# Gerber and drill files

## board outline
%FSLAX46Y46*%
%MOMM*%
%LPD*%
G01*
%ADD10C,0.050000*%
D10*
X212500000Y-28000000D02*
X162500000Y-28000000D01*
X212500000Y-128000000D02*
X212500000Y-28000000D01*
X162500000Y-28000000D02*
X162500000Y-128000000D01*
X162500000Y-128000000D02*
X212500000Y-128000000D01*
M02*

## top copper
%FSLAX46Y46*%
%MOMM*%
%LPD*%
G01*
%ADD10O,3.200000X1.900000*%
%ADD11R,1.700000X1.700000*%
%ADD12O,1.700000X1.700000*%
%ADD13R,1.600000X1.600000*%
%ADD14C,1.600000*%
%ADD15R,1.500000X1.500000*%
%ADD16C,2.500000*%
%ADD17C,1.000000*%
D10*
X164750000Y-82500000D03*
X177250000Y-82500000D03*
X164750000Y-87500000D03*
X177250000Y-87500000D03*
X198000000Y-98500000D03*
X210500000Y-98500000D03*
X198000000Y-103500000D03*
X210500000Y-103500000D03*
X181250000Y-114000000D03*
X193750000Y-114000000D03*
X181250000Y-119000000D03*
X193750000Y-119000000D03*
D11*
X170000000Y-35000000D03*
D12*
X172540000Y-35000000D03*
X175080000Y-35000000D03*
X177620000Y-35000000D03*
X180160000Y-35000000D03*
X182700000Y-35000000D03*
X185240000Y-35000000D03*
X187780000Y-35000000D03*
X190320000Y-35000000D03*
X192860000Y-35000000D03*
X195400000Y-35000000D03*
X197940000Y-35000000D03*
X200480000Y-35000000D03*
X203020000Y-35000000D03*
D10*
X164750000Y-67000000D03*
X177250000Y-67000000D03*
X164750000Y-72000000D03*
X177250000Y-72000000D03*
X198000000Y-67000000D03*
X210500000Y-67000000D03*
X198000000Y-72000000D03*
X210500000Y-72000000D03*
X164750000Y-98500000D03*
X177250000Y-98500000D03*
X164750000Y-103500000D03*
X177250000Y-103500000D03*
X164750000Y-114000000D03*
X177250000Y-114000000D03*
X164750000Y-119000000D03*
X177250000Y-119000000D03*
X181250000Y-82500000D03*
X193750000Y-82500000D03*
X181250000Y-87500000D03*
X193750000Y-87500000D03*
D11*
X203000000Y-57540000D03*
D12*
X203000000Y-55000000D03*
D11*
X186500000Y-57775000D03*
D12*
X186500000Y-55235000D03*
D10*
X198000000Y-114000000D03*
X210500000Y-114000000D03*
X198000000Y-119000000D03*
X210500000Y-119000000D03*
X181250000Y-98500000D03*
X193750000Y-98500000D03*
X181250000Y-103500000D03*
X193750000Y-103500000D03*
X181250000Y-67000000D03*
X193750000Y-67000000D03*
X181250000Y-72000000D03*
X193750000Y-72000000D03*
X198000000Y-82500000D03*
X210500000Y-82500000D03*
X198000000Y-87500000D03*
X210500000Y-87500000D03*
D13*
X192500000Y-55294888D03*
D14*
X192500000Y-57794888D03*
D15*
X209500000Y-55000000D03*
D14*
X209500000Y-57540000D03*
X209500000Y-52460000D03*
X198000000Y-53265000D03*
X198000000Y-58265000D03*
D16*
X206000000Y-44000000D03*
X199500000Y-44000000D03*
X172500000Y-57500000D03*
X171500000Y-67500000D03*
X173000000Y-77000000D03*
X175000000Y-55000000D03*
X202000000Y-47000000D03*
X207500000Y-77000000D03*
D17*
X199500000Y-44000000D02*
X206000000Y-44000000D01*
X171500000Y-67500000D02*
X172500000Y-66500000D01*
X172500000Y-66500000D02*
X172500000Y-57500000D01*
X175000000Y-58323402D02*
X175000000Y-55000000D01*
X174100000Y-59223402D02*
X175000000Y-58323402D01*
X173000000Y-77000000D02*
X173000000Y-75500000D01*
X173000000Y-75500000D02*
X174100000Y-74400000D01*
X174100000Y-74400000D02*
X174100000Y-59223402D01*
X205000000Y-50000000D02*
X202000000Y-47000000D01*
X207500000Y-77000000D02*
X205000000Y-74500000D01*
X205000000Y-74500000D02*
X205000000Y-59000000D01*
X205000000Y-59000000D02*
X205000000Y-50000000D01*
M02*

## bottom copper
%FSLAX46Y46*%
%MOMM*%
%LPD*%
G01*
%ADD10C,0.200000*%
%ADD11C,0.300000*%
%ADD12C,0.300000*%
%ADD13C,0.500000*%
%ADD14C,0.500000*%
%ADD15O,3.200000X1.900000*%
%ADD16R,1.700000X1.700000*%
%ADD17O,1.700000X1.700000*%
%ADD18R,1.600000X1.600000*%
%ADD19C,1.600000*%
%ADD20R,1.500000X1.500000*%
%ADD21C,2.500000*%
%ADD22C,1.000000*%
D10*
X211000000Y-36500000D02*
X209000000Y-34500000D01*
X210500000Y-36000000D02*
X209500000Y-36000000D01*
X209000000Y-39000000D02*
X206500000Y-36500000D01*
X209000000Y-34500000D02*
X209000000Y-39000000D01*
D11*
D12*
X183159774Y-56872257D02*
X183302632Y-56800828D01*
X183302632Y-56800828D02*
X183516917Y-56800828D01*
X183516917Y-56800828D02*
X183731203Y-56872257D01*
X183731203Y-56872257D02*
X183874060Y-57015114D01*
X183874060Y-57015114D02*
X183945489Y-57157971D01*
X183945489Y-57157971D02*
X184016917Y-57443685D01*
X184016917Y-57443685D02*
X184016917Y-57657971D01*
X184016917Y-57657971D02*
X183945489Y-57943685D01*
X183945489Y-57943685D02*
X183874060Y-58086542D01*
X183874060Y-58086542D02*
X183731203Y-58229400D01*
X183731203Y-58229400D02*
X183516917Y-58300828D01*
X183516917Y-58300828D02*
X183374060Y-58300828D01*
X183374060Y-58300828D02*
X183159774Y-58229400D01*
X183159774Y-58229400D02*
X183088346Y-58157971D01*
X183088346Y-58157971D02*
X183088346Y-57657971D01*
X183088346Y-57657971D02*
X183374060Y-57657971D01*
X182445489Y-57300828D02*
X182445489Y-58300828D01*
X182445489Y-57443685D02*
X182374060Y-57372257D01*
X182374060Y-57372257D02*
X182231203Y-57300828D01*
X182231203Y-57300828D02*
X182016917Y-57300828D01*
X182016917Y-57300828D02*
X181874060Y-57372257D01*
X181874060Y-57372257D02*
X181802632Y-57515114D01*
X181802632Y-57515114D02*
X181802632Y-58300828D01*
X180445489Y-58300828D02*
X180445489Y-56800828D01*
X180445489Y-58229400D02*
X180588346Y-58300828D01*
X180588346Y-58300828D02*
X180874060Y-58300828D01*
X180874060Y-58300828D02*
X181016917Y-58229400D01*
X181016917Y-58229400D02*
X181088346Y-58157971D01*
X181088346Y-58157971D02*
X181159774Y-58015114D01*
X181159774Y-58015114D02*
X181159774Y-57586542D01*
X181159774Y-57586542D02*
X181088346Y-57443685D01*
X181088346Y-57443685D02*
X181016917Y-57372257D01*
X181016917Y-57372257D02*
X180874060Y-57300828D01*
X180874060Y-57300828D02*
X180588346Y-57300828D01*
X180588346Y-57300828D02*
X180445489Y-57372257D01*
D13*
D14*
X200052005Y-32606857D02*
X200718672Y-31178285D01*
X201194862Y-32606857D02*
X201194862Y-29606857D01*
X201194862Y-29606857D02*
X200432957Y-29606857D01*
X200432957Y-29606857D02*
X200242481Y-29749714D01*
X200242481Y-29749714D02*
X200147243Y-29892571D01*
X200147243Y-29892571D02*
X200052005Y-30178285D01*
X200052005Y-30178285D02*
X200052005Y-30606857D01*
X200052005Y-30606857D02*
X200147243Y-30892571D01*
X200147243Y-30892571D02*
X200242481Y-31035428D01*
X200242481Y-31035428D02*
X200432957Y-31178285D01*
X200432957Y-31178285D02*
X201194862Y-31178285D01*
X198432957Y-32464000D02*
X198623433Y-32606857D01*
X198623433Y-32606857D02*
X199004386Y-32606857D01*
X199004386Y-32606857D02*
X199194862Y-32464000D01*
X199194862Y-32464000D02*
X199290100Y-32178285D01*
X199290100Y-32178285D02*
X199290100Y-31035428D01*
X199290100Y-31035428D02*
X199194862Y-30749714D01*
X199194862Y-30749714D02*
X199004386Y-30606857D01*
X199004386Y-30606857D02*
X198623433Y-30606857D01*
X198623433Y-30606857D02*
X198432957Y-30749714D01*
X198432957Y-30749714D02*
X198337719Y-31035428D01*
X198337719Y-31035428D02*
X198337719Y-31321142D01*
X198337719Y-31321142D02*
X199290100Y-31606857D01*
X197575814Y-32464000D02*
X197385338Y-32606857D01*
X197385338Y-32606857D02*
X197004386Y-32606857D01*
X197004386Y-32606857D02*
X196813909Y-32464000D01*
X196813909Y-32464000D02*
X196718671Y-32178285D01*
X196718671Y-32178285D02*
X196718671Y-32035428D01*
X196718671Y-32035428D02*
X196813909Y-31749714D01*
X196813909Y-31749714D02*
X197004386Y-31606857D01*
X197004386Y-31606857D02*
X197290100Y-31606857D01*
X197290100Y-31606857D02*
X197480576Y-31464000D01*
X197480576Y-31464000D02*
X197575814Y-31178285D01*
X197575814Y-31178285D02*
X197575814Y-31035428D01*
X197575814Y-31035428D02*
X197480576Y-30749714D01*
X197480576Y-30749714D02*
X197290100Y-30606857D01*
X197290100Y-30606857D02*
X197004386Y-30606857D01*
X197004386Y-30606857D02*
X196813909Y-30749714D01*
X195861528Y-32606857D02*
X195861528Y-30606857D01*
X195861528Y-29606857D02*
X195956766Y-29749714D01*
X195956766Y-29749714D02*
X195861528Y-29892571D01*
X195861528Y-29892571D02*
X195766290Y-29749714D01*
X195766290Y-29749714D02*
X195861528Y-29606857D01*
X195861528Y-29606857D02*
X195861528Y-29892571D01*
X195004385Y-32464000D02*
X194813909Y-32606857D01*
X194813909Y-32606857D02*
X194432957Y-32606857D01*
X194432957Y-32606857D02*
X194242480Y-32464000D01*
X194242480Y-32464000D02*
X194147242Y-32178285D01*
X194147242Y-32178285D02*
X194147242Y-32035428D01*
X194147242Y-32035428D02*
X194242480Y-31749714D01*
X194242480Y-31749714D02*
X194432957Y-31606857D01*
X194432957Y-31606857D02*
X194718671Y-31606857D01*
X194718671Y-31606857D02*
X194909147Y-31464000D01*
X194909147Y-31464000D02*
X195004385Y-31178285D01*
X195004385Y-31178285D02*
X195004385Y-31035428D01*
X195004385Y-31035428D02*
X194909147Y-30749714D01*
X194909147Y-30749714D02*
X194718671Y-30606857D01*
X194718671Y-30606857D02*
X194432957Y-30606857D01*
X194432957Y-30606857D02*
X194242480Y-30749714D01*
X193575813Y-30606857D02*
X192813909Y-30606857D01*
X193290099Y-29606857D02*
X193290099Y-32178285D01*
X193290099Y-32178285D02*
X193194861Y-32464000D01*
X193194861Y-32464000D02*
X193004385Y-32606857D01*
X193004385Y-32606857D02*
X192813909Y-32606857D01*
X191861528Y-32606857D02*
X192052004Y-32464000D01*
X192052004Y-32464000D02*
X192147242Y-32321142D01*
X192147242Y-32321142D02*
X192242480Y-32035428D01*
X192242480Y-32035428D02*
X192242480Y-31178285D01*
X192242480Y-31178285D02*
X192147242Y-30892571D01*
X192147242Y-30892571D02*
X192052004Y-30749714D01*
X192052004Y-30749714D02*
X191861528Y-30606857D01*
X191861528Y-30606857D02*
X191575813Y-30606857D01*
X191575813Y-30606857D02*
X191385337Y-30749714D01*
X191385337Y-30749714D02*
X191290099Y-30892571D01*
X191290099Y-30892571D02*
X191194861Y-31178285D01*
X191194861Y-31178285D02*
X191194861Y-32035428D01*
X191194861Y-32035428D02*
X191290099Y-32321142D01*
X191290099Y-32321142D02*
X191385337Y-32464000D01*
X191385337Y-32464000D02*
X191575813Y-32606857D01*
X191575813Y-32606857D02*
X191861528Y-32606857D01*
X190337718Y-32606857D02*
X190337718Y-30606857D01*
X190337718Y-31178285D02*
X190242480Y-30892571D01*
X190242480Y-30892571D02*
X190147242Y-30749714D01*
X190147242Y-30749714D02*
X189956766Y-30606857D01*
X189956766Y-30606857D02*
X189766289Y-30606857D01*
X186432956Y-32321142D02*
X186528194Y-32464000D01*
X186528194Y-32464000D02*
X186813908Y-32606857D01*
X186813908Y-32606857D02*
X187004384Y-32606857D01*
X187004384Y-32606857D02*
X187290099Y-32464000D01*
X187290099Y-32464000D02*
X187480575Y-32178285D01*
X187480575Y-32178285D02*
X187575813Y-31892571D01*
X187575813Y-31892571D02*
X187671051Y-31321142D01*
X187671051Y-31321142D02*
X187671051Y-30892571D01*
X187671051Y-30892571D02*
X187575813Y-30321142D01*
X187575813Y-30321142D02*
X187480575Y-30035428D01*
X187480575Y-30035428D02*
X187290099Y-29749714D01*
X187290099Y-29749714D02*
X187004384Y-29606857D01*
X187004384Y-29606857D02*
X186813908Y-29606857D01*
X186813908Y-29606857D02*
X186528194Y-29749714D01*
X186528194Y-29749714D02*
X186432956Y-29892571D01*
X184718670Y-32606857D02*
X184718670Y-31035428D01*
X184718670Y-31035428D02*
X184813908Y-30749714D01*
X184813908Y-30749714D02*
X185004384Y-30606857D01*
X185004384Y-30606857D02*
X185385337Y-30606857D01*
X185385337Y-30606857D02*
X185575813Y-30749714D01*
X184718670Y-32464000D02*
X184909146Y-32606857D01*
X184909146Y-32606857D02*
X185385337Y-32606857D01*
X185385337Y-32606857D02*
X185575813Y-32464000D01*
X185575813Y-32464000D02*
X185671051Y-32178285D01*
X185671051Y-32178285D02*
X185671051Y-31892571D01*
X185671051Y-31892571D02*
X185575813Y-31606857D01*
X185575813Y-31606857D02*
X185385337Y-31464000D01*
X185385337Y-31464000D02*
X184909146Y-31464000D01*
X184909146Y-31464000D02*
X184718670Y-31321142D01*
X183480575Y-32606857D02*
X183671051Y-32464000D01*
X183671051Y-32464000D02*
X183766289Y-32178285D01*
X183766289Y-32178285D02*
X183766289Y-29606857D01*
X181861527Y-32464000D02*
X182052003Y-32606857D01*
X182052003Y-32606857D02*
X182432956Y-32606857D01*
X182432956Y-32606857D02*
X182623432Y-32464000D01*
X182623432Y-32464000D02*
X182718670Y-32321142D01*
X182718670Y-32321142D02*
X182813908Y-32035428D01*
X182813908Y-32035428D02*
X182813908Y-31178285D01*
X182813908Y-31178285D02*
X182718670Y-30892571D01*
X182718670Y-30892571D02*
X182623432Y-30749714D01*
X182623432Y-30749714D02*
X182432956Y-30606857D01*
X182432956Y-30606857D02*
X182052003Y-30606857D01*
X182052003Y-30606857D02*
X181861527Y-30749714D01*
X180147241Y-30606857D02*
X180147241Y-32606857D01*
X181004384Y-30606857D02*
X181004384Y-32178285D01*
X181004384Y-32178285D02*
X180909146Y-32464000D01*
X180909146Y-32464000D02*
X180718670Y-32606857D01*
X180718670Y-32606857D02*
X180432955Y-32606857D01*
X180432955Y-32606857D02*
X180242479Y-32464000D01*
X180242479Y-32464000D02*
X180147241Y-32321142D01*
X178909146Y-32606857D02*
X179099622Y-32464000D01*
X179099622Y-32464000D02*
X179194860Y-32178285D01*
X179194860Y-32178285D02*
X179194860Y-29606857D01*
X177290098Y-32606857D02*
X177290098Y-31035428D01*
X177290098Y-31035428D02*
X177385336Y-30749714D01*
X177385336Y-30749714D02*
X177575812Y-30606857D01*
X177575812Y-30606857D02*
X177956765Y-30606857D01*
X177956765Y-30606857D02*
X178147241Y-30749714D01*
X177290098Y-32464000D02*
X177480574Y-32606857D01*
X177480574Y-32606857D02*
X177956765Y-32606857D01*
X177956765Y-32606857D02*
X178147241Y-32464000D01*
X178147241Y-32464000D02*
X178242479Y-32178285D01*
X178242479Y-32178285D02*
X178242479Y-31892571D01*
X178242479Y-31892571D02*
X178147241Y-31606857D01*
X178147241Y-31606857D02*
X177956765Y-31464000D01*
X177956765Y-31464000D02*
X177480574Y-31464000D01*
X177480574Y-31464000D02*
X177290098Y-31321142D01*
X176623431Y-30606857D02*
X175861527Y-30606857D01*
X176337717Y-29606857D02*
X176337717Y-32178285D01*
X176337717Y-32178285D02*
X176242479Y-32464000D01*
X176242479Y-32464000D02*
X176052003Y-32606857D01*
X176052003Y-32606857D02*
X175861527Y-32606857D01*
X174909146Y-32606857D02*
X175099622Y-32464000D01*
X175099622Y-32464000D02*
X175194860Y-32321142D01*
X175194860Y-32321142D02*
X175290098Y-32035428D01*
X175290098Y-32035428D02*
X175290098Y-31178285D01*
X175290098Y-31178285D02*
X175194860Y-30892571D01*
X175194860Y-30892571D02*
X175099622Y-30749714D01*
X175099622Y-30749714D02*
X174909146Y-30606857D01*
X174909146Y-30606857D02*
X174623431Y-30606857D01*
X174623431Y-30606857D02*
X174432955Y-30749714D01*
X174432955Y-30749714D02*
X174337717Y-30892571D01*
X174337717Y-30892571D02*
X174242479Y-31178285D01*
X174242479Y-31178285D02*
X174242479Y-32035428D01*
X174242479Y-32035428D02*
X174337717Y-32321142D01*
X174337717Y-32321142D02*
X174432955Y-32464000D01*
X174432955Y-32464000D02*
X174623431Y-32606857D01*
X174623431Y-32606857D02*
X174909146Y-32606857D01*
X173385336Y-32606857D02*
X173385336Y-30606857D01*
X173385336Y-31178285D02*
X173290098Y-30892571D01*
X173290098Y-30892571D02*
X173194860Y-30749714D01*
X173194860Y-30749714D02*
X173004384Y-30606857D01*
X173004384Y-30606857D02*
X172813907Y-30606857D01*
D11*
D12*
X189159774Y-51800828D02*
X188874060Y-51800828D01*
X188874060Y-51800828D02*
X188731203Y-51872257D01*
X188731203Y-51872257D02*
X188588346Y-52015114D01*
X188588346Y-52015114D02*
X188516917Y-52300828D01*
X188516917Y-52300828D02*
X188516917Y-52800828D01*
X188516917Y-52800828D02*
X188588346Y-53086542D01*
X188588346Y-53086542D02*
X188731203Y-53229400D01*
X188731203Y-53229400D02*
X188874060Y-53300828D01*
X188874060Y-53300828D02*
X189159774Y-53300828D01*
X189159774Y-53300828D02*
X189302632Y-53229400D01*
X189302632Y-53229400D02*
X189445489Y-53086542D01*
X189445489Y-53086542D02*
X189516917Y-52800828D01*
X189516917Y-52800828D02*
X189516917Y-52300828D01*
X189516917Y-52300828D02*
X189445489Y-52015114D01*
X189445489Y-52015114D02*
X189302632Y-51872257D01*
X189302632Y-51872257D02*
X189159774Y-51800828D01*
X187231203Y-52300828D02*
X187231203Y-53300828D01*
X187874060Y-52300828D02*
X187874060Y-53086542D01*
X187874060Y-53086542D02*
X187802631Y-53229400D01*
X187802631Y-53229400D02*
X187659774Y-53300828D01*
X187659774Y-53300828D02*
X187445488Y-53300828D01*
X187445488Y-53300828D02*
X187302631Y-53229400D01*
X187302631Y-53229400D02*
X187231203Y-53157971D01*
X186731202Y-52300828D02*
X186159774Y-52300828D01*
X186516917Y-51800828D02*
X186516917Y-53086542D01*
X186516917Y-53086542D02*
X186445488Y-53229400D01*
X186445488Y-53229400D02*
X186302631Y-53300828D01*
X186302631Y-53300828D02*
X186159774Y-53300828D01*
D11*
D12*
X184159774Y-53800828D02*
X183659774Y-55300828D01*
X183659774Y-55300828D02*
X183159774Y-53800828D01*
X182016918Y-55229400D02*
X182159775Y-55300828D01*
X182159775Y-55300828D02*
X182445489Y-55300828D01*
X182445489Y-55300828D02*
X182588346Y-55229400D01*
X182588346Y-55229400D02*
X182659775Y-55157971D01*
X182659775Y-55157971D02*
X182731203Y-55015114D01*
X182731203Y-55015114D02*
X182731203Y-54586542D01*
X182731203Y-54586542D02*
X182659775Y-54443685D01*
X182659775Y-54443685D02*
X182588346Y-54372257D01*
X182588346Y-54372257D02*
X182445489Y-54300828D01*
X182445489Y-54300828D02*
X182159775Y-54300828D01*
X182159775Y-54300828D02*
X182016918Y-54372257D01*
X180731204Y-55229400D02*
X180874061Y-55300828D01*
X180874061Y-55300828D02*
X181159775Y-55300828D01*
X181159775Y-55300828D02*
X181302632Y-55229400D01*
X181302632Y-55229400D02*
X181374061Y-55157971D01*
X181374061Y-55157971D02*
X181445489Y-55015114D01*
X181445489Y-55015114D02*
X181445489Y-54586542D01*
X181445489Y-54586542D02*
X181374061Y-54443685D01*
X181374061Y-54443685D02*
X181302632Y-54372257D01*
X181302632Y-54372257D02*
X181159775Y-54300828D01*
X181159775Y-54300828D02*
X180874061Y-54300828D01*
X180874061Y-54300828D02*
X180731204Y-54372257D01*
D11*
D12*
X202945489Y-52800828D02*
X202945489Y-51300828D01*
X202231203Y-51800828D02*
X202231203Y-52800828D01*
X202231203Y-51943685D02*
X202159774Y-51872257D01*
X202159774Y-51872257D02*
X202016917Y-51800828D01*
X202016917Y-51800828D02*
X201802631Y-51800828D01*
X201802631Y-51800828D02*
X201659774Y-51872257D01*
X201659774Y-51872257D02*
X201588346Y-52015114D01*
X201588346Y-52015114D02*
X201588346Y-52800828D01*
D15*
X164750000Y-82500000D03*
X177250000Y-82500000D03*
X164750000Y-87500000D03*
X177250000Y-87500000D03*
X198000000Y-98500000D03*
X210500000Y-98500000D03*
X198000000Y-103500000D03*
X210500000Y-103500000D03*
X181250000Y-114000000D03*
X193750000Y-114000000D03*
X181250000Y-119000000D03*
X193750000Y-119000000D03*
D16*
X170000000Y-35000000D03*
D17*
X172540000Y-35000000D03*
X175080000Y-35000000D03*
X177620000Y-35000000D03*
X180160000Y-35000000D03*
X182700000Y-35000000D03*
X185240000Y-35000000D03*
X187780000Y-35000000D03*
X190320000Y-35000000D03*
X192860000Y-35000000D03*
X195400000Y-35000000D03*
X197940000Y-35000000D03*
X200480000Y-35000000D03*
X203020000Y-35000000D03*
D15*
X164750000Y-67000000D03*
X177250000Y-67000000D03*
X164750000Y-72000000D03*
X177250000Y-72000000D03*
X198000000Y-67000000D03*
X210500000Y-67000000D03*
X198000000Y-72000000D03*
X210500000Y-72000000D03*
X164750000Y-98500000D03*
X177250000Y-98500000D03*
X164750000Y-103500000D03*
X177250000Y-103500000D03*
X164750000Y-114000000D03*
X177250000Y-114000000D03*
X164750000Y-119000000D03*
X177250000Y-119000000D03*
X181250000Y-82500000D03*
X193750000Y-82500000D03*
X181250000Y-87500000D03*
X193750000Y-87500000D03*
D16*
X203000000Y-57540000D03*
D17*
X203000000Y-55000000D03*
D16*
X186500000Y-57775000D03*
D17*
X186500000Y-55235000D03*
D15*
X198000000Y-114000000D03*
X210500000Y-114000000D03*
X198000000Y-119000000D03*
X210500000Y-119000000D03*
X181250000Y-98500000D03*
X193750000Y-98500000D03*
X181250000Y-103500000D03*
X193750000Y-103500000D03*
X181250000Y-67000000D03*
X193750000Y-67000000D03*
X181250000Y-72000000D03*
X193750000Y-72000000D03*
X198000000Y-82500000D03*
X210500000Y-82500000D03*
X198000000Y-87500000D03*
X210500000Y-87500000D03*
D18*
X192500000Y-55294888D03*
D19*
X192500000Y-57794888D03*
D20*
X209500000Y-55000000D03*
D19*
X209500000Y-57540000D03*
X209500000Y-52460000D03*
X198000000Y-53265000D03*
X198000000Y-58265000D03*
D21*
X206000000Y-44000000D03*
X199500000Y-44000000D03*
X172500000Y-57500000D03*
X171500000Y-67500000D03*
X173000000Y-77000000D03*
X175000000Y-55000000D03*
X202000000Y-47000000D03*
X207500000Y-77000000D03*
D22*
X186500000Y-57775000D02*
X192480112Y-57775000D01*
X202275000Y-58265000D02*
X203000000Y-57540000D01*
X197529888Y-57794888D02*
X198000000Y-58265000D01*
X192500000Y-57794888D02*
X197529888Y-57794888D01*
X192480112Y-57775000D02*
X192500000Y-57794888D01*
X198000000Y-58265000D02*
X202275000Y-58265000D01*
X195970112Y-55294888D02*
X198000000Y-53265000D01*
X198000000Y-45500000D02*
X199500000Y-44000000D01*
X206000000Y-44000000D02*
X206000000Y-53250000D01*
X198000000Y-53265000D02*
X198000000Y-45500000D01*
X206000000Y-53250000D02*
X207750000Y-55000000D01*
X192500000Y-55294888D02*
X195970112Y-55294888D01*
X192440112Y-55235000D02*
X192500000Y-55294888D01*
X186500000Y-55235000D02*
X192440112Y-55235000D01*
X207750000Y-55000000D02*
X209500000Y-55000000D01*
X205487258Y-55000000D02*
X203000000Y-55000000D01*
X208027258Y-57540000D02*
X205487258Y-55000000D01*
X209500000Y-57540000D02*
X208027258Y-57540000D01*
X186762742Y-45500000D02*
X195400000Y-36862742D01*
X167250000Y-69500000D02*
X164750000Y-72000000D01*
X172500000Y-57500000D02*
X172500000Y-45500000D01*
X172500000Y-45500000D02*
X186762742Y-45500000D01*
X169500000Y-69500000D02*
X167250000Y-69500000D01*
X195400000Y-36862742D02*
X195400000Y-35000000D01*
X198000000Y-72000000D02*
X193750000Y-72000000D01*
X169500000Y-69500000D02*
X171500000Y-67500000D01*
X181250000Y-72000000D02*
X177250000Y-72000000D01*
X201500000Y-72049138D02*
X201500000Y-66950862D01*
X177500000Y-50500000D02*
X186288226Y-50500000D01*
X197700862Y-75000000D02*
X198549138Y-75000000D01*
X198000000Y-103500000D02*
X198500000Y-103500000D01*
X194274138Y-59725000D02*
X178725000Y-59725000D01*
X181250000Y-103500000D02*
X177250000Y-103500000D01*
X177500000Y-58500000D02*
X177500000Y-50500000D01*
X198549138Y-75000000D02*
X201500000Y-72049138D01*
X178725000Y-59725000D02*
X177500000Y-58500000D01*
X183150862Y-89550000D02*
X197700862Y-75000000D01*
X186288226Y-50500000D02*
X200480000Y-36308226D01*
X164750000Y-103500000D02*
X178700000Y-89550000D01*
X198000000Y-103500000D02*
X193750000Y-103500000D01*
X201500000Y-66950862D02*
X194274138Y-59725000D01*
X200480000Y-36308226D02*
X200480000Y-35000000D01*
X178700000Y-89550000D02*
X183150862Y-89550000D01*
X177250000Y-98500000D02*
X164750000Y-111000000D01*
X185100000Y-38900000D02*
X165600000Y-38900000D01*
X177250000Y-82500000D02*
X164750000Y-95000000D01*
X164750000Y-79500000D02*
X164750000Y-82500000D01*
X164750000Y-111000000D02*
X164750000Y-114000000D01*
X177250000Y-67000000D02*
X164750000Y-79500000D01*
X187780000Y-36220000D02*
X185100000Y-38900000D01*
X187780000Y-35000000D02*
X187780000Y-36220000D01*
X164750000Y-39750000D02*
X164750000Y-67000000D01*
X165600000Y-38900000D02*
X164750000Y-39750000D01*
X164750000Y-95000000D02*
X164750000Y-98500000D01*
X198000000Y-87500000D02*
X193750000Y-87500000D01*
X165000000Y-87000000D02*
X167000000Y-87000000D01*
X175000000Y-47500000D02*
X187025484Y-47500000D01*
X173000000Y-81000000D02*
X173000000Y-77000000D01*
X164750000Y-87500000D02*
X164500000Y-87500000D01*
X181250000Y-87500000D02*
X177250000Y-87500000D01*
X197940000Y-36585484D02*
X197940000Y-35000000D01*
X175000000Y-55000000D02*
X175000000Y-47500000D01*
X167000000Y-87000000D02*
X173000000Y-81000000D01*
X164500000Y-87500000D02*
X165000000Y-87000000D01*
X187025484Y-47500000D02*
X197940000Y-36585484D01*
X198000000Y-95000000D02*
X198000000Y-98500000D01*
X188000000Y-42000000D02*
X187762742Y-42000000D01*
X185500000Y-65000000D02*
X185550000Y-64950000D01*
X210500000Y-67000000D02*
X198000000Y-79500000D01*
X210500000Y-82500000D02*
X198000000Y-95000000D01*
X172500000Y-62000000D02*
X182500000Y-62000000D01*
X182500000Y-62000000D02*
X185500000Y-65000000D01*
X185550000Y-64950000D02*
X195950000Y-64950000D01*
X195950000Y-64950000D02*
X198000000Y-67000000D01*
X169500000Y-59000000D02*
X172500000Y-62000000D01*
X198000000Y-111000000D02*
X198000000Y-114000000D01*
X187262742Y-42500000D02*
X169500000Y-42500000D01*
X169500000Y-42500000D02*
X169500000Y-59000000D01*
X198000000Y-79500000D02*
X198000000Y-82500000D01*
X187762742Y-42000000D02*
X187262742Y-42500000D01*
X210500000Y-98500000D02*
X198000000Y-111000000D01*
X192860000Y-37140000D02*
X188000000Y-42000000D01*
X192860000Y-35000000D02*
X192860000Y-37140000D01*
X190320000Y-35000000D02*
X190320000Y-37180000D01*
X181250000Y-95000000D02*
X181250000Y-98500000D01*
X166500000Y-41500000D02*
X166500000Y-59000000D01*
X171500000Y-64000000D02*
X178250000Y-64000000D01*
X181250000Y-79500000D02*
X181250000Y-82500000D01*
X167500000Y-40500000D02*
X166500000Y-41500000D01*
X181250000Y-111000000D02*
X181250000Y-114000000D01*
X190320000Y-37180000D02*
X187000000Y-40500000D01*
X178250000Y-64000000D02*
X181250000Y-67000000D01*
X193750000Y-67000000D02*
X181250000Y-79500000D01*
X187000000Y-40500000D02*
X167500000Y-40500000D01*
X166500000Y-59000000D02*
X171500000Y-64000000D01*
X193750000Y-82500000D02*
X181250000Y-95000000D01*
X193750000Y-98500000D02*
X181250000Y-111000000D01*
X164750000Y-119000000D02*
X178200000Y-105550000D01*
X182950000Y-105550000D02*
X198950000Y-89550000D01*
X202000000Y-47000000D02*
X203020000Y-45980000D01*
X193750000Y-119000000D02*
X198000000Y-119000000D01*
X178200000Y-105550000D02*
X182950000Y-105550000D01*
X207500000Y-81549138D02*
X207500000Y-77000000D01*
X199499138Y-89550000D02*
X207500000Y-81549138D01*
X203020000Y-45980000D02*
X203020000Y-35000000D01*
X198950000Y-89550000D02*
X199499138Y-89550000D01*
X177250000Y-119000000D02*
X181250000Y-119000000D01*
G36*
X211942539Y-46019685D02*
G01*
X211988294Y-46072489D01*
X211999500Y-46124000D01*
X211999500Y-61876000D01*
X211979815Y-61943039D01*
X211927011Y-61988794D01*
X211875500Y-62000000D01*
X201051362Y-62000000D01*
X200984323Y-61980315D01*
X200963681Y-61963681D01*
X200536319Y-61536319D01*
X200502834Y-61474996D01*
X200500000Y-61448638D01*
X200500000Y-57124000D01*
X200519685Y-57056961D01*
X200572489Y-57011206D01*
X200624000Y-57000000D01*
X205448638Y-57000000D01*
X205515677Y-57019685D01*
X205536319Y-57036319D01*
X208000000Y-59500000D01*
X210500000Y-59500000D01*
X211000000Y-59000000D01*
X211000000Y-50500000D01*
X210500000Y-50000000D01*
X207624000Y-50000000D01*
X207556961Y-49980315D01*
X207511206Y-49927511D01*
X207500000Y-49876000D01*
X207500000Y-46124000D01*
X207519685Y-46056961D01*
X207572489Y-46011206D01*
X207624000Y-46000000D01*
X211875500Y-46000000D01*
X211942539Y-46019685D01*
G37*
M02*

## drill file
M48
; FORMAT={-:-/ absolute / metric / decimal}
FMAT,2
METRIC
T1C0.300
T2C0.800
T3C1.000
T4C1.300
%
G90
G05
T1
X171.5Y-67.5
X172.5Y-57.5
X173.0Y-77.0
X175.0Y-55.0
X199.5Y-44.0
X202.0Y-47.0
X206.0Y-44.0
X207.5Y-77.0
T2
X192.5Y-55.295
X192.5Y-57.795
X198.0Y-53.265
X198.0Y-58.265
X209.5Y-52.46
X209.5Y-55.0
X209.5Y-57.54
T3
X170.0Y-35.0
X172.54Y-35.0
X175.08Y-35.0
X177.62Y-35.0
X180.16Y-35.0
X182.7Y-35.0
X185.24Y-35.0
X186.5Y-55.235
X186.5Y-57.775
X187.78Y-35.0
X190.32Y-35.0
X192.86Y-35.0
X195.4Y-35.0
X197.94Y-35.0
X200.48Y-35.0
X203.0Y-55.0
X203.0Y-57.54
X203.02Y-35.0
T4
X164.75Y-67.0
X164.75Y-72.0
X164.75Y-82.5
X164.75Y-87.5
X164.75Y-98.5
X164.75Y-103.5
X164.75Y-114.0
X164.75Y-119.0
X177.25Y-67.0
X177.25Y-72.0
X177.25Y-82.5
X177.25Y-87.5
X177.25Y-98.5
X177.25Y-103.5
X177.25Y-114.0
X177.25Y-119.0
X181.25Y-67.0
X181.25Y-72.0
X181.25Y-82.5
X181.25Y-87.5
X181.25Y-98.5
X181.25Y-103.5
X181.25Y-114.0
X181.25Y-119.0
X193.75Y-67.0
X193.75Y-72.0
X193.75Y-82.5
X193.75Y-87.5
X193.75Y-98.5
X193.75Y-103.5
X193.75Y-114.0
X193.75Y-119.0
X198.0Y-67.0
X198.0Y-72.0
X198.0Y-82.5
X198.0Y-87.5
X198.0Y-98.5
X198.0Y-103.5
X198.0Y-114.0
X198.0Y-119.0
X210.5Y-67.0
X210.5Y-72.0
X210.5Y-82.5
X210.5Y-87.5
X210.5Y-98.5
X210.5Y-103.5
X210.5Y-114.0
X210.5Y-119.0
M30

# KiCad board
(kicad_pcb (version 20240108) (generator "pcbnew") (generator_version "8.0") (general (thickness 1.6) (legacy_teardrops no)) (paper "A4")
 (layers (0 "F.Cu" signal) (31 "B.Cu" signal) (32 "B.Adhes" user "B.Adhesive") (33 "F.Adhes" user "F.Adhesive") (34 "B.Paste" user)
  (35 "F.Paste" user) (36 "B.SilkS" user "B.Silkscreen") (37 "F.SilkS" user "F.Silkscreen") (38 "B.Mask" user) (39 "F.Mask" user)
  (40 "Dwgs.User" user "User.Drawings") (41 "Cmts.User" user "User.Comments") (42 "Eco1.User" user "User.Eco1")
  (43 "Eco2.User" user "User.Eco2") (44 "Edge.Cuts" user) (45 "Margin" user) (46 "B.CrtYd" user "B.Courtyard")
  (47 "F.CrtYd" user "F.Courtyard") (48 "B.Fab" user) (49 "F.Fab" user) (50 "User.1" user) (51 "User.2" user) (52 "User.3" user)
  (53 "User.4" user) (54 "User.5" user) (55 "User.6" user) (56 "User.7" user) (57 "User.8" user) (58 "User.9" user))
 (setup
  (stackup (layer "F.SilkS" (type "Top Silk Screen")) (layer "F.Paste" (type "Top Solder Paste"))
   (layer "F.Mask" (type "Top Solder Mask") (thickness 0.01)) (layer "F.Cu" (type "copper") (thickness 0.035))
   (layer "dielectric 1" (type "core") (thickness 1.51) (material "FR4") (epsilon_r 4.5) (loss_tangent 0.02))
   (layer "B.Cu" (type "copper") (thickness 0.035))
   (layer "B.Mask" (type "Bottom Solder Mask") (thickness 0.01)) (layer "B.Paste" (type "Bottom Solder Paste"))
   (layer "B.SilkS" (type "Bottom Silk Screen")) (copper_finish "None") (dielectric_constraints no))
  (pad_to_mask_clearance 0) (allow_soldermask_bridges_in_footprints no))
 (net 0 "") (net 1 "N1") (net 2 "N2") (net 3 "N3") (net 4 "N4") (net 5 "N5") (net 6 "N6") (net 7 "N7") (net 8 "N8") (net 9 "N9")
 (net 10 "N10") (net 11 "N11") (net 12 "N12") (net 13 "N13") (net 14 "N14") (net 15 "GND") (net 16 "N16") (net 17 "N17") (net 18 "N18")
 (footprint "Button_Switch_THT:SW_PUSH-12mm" (layer "F.Cu") (at 164.75 82.5)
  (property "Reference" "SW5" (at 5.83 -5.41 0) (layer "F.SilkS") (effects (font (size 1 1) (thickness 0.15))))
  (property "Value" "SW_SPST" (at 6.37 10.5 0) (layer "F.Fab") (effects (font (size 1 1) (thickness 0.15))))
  (pad "1" thru_hole oval (at 0 0) (size 3.2 1.9) (drill 1.3) (layers "*.Cu" "*.Mask") (remove_unused_layers no) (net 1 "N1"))
  (pad "1" thru_hole oval (at 12.5 0) (size 3.2 1.9) (drill 1.3) (layers "*.Cu" "*.Mask") (remove_unused_layers no) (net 1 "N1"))
  (pad "2" thru_hole oval (at 0 5) (size 3.2 1.9) (drill 1.3) (layers "*.Cu" "*.Mask") (remove_unused_layers no) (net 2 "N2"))
  (pad "2" thru_hole oval (at 12.5 5) (size 3.2 1.9) (drill 1.3) (layers "*.Cu" "*.Mask") (remove_unused_layers no) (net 2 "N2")))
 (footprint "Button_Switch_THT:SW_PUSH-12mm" (layer "F.Cu") (at 198 98.5)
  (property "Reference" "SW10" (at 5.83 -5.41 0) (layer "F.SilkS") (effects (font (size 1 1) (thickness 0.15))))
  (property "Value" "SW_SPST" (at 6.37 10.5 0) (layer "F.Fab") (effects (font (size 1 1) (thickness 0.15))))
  (pad "1" thru_hole oval (at 0 0) (size 3.2 1.9) (drill 1.3) (layers "*.Cu" "*.Mask") (remove_unused_layers no) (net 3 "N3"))
  (pad "1" thru_hole oval (at 12.5 0) (size 3.2 1.9) (drill 1.3) (layers "*.Cu" "*.Mask") (remove_unused_layers no) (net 3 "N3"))
  (pad "2" thru_hole oval (at 0 5) (size 3.2 1.9) (drill 1.3) (layers "*.Cu" "*.Mask") (remove_unused_layers no) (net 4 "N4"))
  (pad "2" thru_hole oval (at 12.5 5) (size 3.2 1.9) (drill 1.3) (layers "*.Cu" "*.Mask") (remove_unused_layers no) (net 4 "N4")))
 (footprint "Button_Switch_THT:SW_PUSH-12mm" (layer "F.Cu") (at 181.25 114)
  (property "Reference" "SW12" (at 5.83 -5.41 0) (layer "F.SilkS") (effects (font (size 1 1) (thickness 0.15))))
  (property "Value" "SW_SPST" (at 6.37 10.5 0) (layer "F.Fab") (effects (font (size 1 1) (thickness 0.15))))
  (pad "1" thru_hole oval (at 0 0) (size 3.2 1.9) (drill 1.3) (layers "*.Cu" "*.Mask") (remove_unused_layers no) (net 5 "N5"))
  (pad "1" thru_hole oval (at 12.5 0) (size 3.2 1.9) (drill 1.3) (layers "*.Cu" "*.Mask") (remove_unused_layers no) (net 5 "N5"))
  (pad "2" thru_hole oval (at 0 5) (size 3.2 1.9) (drill 1.3) (layers "*.Cu" "*.Mask") (remove_unused_layers no) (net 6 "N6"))
  (pad "2" thru_hole oval (at 12.5 5) (size 3.2 1.9) (drill 1.3) (layers "*.Cu" "*.Mask") (remove_unused_layers no) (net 6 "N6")))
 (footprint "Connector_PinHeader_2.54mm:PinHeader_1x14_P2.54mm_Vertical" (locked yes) (layer "F.Cu") (at 170 35 90)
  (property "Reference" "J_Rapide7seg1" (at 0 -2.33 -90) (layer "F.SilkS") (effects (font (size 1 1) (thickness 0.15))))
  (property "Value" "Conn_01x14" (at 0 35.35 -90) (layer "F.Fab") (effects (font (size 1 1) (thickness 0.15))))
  (pad "1" thru_hole rect (at 0 0 90) (size 1.7 1.7) (drill 1) (layers "*.Cu" "*.Mask") (remove_unused_layers no) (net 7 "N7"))
  (pad "2" thru_hole oval (at 0 2.54 90) (size 1.7 1.7) (drill 1) (layers "*.Cu" "*.Mask") (remove_unused_layers no) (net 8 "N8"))
  (pad "3" thru_hole oval (at 0 5.08 90) (size 1.7 1.7) (drill 1) (layers "*.Cu" "*.Mask") (remove_unused_layers no) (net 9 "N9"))
  (pad "4" thru_hole oval (at 0 7.62 90) (size 1.7 1.7) (drill 1) (layers "*.Cu" "*.Mask") (remove_unused_layers no) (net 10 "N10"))
  (pad "5" thru_hole oval (at 0 10.16 90) (size 1.7 1.7) (drill 1) (layers "*.Cu" "*.Mask") (remove_unused_layers no) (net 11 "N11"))
  (pad "6" thru_hole oval (at 0 12.7 90) (size 1.7 1.7) (drill 1) (layers "*.Cu" "*.Mask") (remove_unused_layers no) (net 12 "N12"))
  (pad "7" thru_hole oval (at 0 15.24 90) (size 1.7 1.7) (drill 1) (layers "*.Cu" "*.Mask") (remove_unused_layers no) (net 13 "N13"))
  (pad "8" thru_hole oval (at 0 17.78 90) (size 1.7 1.7) (drill 1) (layers "*.Cu" "*.Mask") (remove_unused_layers no) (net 1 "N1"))
  (pad "9" thru_hole oval (at 0 20.32 90) (size 1.7 1.7) (drill 1) (layers "*.Cu" "*.Mask") (remove_unused_layers no) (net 5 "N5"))
  (pad "10" thru_hole oval (at 0 22.86 90) (size 1.7 1.7) (drill 1) (layers "*.Cu" "*.Mask") (remove_unused_layers no) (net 3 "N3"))
  (pad "11" thru_hole oval (at 0 25.4 90) (size 1.7 1.7) (drill 1) (layers "*.Cu" "*.Mask") (remove_unused_layers no) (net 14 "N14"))
  (pad "12" thru_hole oval (at 0 27.94 90) (size 1.7 1.7) (drill 1) (layers "*.Cu" "*.Mask") (remove_unused_layers no) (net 2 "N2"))
  (pad "13" thru_hole oval (at 0 30.48 90) (size 1.7 1.7) (drill 1) (layers "*.Cu" "*.Mask") (remove_unused_layers no) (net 4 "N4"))
  (pad "14" thru_hole oval (at 0 33.02 90) (size 1.7 1.7) (drill 1) (layers "*.Cu" "*.Mask") (remove_unused_layers no) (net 6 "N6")))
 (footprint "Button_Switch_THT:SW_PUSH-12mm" (layer "F.Cu") (at 164.75 67)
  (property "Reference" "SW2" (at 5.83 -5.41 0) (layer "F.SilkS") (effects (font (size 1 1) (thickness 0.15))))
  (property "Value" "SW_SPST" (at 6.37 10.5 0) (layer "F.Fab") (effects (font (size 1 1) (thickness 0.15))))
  (pad "1" thru_hole oval (at 0 0) (size 3.2 1.9) (drill 1.3) (layers "*.Cu" "*.Mask") (remove_unused_layers no) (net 1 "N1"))
  (pad "1" thru_hole oval (at 12.5 0) (size 3.2 1.9) (drill 1.3) (layers "*.Cu" "*.Mask") (remove_unused_layers no) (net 1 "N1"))
  (pad "2" thru_hole oval (at 0 5) (size 3.2 1.9) (drill 1.3) (layers "*.Cu" "*.Mask") (remove_unused_layers no) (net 14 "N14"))
  (pad "2" thru_hole oval (at 12.5 5) (size 3.2 1.9) (drill 1.3) (layers "*.Cu" "*.Mask") (remove_unused_layers no) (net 14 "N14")))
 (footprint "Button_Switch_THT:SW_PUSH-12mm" (layer "F.Cu") (at 198 67)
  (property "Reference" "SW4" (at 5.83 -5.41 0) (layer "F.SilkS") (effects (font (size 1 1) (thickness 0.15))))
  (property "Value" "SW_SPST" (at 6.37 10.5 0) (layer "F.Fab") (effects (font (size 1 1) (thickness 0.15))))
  (pad "1" thru_hole oval (at 0 0) (size 3.2 1.9) (drill 1.3) (layers "*.Cu" "*.Mask") (remove_unused_layers no) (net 3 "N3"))
  (pad "1" thru_hole oval (at 12.5 0) (size 3.2 1.9) (drill 1.3) (layers "*.Cu" "*.Mask") (remove_unused_layers no) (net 3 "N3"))
  (pad "2" thru_hole oval (at 0 5) (size 3.2 1.9) (drill 1.3) (layers "*.Cu" "*.Mask") (remove_unused_layers no) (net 14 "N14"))
  (pad "2" thru_hole oval (at 12.5 5) (size 3.2 1.9) (drill 1.3) (layers "*.Cu" "*.Mask") (remove_unused_layers no) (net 14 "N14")))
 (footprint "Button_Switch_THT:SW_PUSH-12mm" (layer "F.Cu") (at 164.75 98.5)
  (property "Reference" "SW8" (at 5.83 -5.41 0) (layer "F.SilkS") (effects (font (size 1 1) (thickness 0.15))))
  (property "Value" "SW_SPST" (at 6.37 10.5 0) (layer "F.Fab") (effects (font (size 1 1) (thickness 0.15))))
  (pad "1" thru_hole oval (at 0 0) (size 3.2 1.9) (drill 1.3) (layers "*.Cu" "*.Mask") (remove_unused_layers no) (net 1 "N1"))
  (pad "1" thru_hole oval (at 12.5 0) (size 3.2 1.9) (drill 1.3) (layers "*.Cu" "*.Mask") (remove_unused_layers no) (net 1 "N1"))
  (pad "2" thru_hole oval (at 0 5) (size 3.2 1.9) (drill 1.3) (layers "*.Cu" "*.Mask") (remove_unused_layers no) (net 4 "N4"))
  (pad "2" thru_hole oval (at 12.5 5) (size 3.2 1.9) (drill 1.3) (layers "*.Cu" "*.Mask") (remove_unused_layers no) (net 4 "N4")))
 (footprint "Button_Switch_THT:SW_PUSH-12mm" (layer "F.Cu") (at 164.75 114)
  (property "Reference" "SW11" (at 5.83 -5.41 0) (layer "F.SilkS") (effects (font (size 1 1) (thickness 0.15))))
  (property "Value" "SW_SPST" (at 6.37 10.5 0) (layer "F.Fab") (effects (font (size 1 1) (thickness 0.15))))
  (pad "1" thru_hole oval (at 0 0) (size 3.2 1.9) (drill 1.3) (layers "*.Cu" "*.Mask") (remove_unused_layers no) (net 1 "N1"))
  (pad "1" thru_hole oval (at 12.5 0) (size 3.2 1.9) (drill 1.3) (layers "*.Cu" "*.Mask") (remove_unused_layers no) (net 1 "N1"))
  (pad "2" thru_hole oval (at 0 5) (size 3.2 1.9) (drill 1.3) (layers "*.Cu" "*.Mask") (remove_unused_layers no) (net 6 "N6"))
  (pad "2" thru_hole oval (at 12.5 5) (size 3.2 1.9) (drill 1.3) (layers "*.Cu" "*.Mask") (remove_unused_layers no) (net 6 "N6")))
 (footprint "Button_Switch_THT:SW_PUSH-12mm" (layer "F.Cu") (at 181.25 82.5)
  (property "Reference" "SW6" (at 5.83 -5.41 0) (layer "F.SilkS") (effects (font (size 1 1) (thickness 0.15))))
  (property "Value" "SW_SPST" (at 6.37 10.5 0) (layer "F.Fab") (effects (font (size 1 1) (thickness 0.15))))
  (pad "1" thru_hole oval (at 0 0) (size 3.2 1.9) (drill 1.3) (layers "*.Cu" "*.Mask") (remove_unused_layers no) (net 5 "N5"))
  (pad "1" thru_hole oval (at 12.5 0) (size 3.2 1.9) (drill 1.3) (layers "*.Cu" "*.Mask") (remove_unused_layers no) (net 5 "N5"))
  (pad "2" thru_hole oval (at 0 5) (size 3.2 1.9) (drill 1.3) (layers "*.Cu" "*.Mask") (remove_unused_layers no) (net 2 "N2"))
  (pad "2" thru_hole oval (at 12.5 5) (size 3.2 1.9) (drill 1.3) (layers "*.Cu" "*.Mask") (remove_unused_layers no) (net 2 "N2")))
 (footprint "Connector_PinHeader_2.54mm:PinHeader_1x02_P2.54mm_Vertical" (layer "F.Cu") (at 203 57.54 180)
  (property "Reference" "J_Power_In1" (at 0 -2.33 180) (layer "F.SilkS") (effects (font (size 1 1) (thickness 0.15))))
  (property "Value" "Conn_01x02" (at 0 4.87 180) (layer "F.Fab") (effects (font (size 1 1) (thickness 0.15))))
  (pad "1" thru_hole rect (at 0 0 180) (size 1.7 1.7) (drill 1) (layers "*.Cu" "*.Mask") (remove_unused_layers no) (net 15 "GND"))
  (pad "2" thru_hole oval (at 0 2.54 180) (size 1.7 1.7) (drill 1) (layers "*.Cu" "*.Mask") (remove_unused_layers no) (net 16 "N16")))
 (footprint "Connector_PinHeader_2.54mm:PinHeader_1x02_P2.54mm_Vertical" (layer "F.Cu") (at 186.5 57.775 180)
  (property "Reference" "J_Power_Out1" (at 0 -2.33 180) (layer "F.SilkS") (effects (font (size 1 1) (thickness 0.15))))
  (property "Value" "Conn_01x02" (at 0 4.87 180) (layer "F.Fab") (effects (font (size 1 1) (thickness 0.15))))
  (pad "1" thru_hole rect (at 0 0 180) (size 1.7 1.7) (drill 1) (layers "*.Cu" "*.Mask") (remove_unused_layers no) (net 15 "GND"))
  (pad "2" thru_hole oval (at 0 2.54 180) (size 1.7 1.7) (drill 1) (layers "*.Cu" "*.Mask") (remove_unused_layers no) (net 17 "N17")))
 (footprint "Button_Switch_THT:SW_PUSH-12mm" (layer "F.Cu") (at 198 114)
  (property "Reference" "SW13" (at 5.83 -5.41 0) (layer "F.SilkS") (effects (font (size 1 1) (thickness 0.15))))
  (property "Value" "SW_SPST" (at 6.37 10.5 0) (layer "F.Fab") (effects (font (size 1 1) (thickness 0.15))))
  (pad "1" thru_hole oval (at 0 0) (size 3.2 1.9) (drill 1.3) (layers "*.Cu" "*.Mask") (remove_unused_layers no) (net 3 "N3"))
  (pad "1" thru_hole oval (at 12.5 0) (size 3.2 1.9) (drill 1.3) (layers "*.Cu" "*.Mask") (remove_unused_layers no) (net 3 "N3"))
  (pad "2" thru_hole oval (at 0 5) (size 3.2 1.9) (drill 1.3) (layers "*.Cu" "*.Mask") (remove_unused_layers no) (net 6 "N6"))
  (pad "2" thru_hole oval (at 12.5 5) (size 3.2 1.9) (drill 1.3) (layers "*.Cu" "*.Mask") (remove_unused_layers no) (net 6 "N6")))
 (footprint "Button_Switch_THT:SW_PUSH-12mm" (layer "F.Cu") (at 181.25 98.5)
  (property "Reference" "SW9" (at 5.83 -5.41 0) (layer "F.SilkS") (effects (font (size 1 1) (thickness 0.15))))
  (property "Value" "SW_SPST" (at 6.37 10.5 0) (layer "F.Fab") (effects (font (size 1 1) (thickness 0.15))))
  (pad "1" thru_hole oval (at 0 0) (size 3.2 1.9) (drill 1.3) (layers "*.Cu" "*.Mask") (remove_unused_layers no) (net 5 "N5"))
  (pad "1" thru_hole oval (at 12.5 0) (size 3.2 1.9) (drill 1.3) (layers "*.Cu" "*.Mask") (remove_unused_layers no) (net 5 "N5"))
  (pad "2" thru_hole oval (at 0 5) (size 3.2 1.9) (drill 1.3) (layers "*.Cu" "*.Mask") (remove_unused_layers no) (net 4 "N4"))
  (pad "2" thru_hole oval (at 12.5 5) (size 3.2 1.9) (drill 1.3) (layers "*.Cu" "*.Mask") (remove_unused_layers no) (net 4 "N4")))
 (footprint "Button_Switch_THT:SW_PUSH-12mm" (layer "F.Cu") (at 181.25 67)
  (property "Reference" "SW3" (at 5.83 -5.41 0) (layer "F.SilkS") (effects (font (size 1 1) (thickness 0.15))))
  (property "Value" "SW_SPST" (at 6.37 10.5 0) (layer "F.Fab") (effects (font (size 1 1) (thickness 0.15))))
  (pad "1" thru_hole oval (at 0 0) (size 3.2 1.9) (drill 1.3) (layers "*.Cu" "*.Mask") (remove_unused_layers no) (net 5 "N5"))
  (pad "1" thru_hole oval (at 12.5 0) (size 3.2 1.9) (drill 1.3) (layers "*.Cu" "*.Mask") (remove_unused_layers no) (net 5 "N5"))
  (pad "2" thru_hole oval (at 0 5) (size 3.2 1.9) (drill 1.3) (layers "*.Cu" "*.Mask") (remove_unused_layers no) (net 14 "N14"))
  (pad "2" thru_hole oval (at 12.5 5) (size 3.2 1.9) (drill 1.3) (layers "*.Cu" "*.Mask") (remove_unused_layers no) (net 14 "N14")))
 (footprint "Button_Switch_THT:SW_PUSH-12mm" (layer "F.Cu") (at 198 82.5)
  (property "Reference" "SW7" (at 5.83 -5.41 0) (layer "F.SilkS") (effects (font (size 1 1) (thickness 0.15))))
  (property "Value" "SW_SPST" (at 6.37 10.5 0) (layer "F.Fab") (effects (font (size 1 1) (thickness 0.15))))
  (pad "1" thru_hole oval (at 0 0) (size 3.2 1.9) (drill 1.3) (layers "*.Cu" "*.Mask") (remove_unused_layers no) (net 3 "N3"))
  (pad "1" thru_hole oval (at 12.5 0) (size 3.2 1.9) (drill 1.3) (layers "*.Cu" "*.Mask") (remove_unused_layers no) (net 3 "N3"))
  (pad "2" thru_hole oval (at 0 5) (size 3.2 1.9) (drill 1.3) (layers "*.Cu" "*.Mask") (remove_unused_layers no) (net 2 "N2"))
  (pad "2" thru_hole oval (at 12.5 5) (size 3.2 1.9) (drill 1.3) (layers "*.Cu" "*.Mask") (remove_unused_layers no) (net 2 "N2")))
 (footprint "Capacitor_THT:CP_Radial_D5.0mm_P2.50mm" (layer "F.Cu") (at 192.5 55.294888 -90)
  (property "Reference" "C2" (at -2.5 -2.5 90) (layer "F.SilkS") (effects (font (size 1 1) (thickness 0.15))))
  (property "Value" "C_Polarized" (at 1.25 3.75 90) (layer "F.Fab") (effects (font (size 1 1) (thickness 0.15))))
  (pad "1" thru_hole rect (at 0 0 270) (size 1.6 1.6) (drill 0.8) (layers "*.Cu" "*.Mask") (remove_unused_layers no) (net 17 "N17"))
  (pad "2" thru_hole circle (at 2.5 0 270) (size 1.6 1.6) (drill 0.8) (layers "*.Cu" "*.Mask") (remove_unused_layers no) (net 15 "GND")))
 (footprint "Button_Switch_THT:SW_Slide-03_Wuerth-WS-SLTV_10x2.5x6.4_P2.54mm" (layer "F.Cu") (at 209.5 55 90)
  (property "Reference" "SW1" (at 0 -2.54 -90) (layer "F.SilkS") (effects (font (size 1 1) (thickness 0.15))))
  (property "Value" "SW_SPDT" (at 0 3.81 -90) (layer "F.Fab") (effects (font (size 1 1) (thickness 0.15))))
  (pad "1" thru_hole rect (at 0 0 90) (size 1.5 1.5) (drill 0.8) (layers "*.Cu" "*.Mask") (remove_unused_layers no) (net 17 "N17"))
  (pad "2" thru_hole circle (at -2.54 0 90) (size 1.6 1.6) (drill 0.8) (layers "*.Cu" "*.Mask") (remove_unused_layers no) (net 16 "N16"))
  (pad "3" thru_hole circle (at 2.54 0 90) (size 1.6 1.6) (drill 0.8) (layers "*.Cu" "*.Mask") (remove_unused_layers no) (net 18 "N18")))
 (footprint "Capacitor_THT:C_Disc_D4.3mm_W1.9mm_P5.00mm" (layer "F.Cu") (at 198 53.265 -90)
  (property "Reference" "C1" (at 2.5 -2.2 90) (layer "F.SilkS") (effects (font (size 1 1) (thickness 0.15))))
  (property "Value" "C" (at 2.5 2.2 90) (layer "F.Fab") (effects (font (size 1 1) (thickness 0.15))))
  (pad "1" thru_hole circle (at 0 0 270) (size 1.6 1.6) (drill 0.8) (layers "*.Cu" "*.Mask") (remove_unused_layers no) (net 17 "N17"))
  (pad "2" thru_hole circle (at 5 0 270) (size 1.6 1.6) (drill 0.8) (layers "*.Cu" "*.Mask") (remove_unused_layers no) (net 15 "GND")))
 (gr_line (start 211 36.5) (end 209 34.5) (stroke (width 0.2) (type default)) (layer "B.Cu"))
 (gr_line (start 210.5 36) (end 209.5 36) (stroke (width 0.2) (type default)) (layer "B.Cu"))
 (gr_line (start 209 39) (end 206.5 36.5) (stroke (width 0.2) (type default)) (layer "B.Cu"))
 (gr_line (start 209 34.5) (end 209 39) (stroke (width 0.2) (type default)) (layer "B.Cu"))
 (gr_line (start 212.5 28) (end 162.5 28) (stroke (width 0.05) (type default)) (layer "Edge.Cuts"))
 (gr_line (start 212.5 128) (end 212.5 28) (stroke (width 0.05) (type default)) (layer "Edge.Cuts"))
 (gr_line (start 162.5 28) (end 162.5 128) (stroke (width 0.05) (type default)) (layer "Edge.Cuts"))
 (gr_line (start 162.5 128) (end 212.5 128) (stroke (width 0.05) (type default)) (layer "Edge.Cuts"))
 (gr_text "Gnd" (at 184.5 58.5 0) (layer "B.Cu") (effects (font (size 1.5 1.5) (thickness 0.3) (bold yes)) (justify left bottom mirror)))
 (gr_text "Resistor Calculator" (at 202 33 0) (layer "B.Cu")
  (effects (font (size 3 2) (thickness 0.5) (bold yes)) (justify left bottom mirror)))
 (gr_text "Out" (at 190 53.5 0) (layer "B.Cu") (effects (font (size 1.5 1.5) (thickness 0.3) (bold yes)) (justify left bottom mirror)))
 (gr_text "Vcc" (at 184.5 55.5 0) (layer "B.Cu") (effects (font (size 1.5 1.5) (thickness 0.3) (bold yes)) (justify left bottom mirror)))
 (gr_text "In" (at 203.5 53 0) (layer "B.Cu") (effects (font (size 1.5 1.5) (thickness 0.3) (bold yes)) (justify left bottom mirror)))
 (segment (start 186.5 57.775) (end 192.480112 57.775) (width 1) (layer "B.Cu") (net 15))
 (segment (start 202.275 58.265) (end 203 57.54) (width 1) (layer "B.Cu") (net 15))
 (segment (start 197.529888 57.794888) (end 198 58.265) (width 1) (layer "B.Cu") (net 15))
 (segment (start 192.5 57.794888) (end 197.529888 57.794888) (width 1) (layer "B.Cu") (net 15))
 (segment (start 192.480112 57.775) (end 192.5 57.794888) (width 1) (layer "B.Cu") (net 15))
 (segment (start 198 58.265) (end 202.275 58.265) (width 1) (layer "B.Cu") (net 15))
 (segment (start 199.5 44) (end 206 44) (width 1) (layer "F.Cu") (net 17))
 (via (at 206 44) (size 2.5) (drill 0.3) (layers "F.Cu" "B.Cu") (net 17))
 (via (at 199.5 44) (size 2.5) (drill 0.3) (layers "F.Cu" "B.Cu") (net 17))
 (segment (start 195.970112 55.294888) (end 198 53.265) (width 1) (layer "B.Cu") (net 17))
 (segment (start 198 45.5) (end 199.5 44) (width 1) (layer "B.Cu") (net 17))
 (segment (start 206 44) (end 206 53.25) (width 1) (layer "B.Cu") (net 17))
 (segment (start 198 53.265) (end 198 45.5) (width 1) (layer "B.Cu") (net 17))
 (segment (start 206 53.25) (end 207.75 55) (width 1) (layer "B.Cu") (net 17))
 (segment (start 192.5 55.294888) (end 195.970112 55.294888) (width 1) (layer "B.Cu") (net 17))
 (segment (start 192.440112 55.235) (end 192.5 55.294888) (width 1) (layer "B.Cu") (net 17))
 (segment (start 186.5 55.235) (end 192.440112 55.235) (width 1) (layer "B.Cu") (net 17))
 (segment (start 207.75 55) (end 209.5 55) (width 1) (layer "B.Cu") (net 17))
 (segment (start 205.487258 55) (end 203 55) (width 1) (layer "B.Cu") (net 16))
 (segment (start 208.027258 57.54) (end 205.487258 55) (width 1) (layer "B.Cu") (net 16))
 (segment (start 209.5 57.54) (end 208.027258 57.54) (width 1) (layer "B.Cu") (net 16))
 (segment (start 171.5 67.5) (end 172.5 66.5) (width 1) (layer "F.Cu") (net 14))
 (segment (start 172.5 66.5) (end 172.5 57.5) (width 1) (layer "F.Cu") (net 14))
 (via (at 172.5 57.5) (size 2.5) (drill 0.3) (layers "F.Cu" "B.Cu") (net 14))
 (via (at 171.5 67.5) (size 2.5) (drill 0.3) (layers "F.Cu" "B.Cu") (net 14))
 (segment (start 186.762742 45.5) (end 195.4 36.862742) (width 1) (layer "B.Cu") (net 14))
 (segment (start 167.25 69.5) (end 164.75 72) (width 1) (layer "B.Cu") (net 14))
 (segment (start 172.5 57.5) (end 172.5 45.5) (width 1) (layer "B.Cu") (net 14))
 (segment (start 172.5 45.5) (end 186.762742 45.5) (width 1) (layer "B.Cu") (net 14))
 (segment (start 169.5 69.5) (end 167.25 69.5) (width 1) (layer "B.Cu") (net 14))
 (segment (start 195.4 36.862742) (end 195.4 35) (width 1) (layer "B.Cu") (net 14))
 (segment (start 198 72) (end 193.75 72) (width 1) (layer "B.Cu") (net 14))
 (segment (start 169.5 69.5) (end 171.5 67.5) (width 1) (layer "B.Cu") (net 14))
 (segment (start 181.25 72) (end 177.25 72) (width 1) (layer "B.Cu") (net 14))
 (segment (start 201.5 72.049138) (end 201.5 66.950862) (width 1) (layer "B.Cu") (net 4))
 (segment (start 177.5 50.5) (end 186.288226 50.5) (width 1) (layer "B.Cu") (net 4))
 (segment (start 197.700862 75) (end 198.549138 75) (width 1) (layer "B.Cu") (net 4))
 (segment (start 198 103.5) (end 198.5 103.5) (width 1) (layer "B.Cu") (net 4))
 (segment (start 194.274138 59.725) (end 178.725 59.725) (width 1) (layer "B.Cu") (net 4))
 (segment (start 181.25 103.5) (end 177.25 103.5) (width 1) (layer "B.Cu") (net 4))
 (segment (start 177.5 58.5) (end 177.5 50.5) (width 1) (layer "B.Cu") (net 4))
 (segment (start 198.549138 75) (end 201.5 72.049138) (width 1) (layer "B.Cu") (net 4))
 (segment (start 178.725 59.725) (end 177.5 58.5) (width 1) (layer "B.Cu") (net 4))
 (segment (start 183.150862 89.55) (end 197.700862 75) (width 1) (layer "B.Cu") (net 4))
 (segment (start 186.288226 50.5) (end 200.48 36.308226) (width 1) (layer "B.Cu") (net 4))
 (segment (start 164.75 103.5) (end 178.7 89.55) (width 1) (layer "B.Cu") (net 4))
 (segment (start 198 103.5) (end 193.75 103.5) (width 1) (layer "B.Cu") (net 4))
 (segment (start 201.5 66.950862) (end 194.274138 59.725) (width 1) (layer "B.Cu") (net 4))
 (segment (start 200.48 36.308226) (end 200.48 35) (width 1) (layer "B.Cu") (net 4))
 (segment (start 178.7 89.55) (end 183.150862 89.55) (width 1) (layer "B.Cu") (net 4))
 (segment (start 177.25 98.5) (end 164.75 111) (width 1) (layer "B.Cu") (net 1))
 (segment (start 185.1 38.9) (end 165.6 38.9) (width 1) (layer "B.Cu") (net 1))
 (segment (start 177.25 82.5) (end 164.75 95) (width 1) (layer "B.Cu") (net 1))
 (segment (start 164.75 79.5) (end 164.75 82.5) (width 1) (layer "B.Cu") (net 1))
 (segment (start 164.75 111) (end 164.75 114) (width 1) (layer "B.Cu") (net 1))
 (segment (start 177.25 67) (end 164.75 79.5) (width 1) (layer "B.Cu") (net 1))
 (segment (start 187.78 36.22) (end 185.1 38.9) (width 1) (layer "B.Cu") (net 1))
 (segment (start 187.78 35) (end 187.78 36.22) (width 1) (layer "B.Cu") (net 1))
 (segment (start 164.75 39.75) (end 164.75 67) (width 1) (layer "B.Cu") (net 1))
 (segment (start 165.6 38.9) (end 164.75 39.75) (width 1) (layer "B.Cu") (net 1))
 (segment (start 164.75 95) (end 164.75 98.5) (width 1) (layer "B.Cu") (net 1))
 (segment (start 175 58.323402) (end 175 55) (width 1) (layer "F.Cu") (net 2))
 (segment (start 174.1 59.223402) (end 175 58.323402) (width 1) (layer "F.Cu") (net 2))
 (segment (start 173 77) (end 173 75.5) (width 1) (layer "F.Cu") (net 2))
 (segment (start 173 75.5) (end 174.1 74.4) (width 1) (layer "F.Cu") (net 2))
 (segment (start 174.1 74.4) (end 174.1 59.223402) (width 1) (layer "F.Cu") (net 2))
 (via (at 173 77) (size 2.5) (drill 0.3) (layers "F.Cu" "B.Cu") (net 2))
 (via (at 175 55) (size 2.5) (drill 0.3) (layers "F.Cu" "B.Cu") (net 2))
 (segment (start 198 87.5) (end 193.75 87.5) (width 1) (layer "B.Cu") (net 2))
 (segment (start 165 87) (end 167 87) (width 1) (layer "B.Cu") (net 2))
 (segment (start 175 47.5) (end 187.025484 47.5) (width 1) (layer "B.Cu") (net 2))
 (segment (start 173 81) (end 173 77) (width 1) (layer "B.Cu") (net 2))
 (segment (start 164.75 87.5) (end 164.5 87.5) (width 1) (layer "B.Cu") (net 2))
 (segment (start 181.25 87.5) (end 177.25 87.5) (width 1) (layer "B.Cu") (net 2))
 (segment (start 197.94 36.585484) (end 197.94 35) (width 1) (layer "B.Cu") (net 2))
 (segment (start 175 55) (end 175 47.5) (width 1) (layer "B.Cu") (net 2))
 (segment (start 167 87) (end 173 81) (width 1) (layer "B.Cu") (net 2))
 (segment (start 164.5 87.5) (end 165 87) (width 1) (layer "B.Cu") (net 2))
 (segment (start 187.025484 47.5) (end 197.94 36.585484) (width 1) (layer "B.Cu") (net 2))
 (segment (start 198 95) (end 198 98.5) (width 1) (layer "B.Cu") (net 3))
 (segment (start 188 42) (end 187.762742 42) (width 1) (layer "B.Cu") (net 3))
 (segment (start 185.5 65) (end 185.55 64.95) (width 1) (layer "B.Cu") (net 3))
 (segment (start 210.5 67) (end 198 79.5) (width 1) (layer "B.Cu") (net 3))
 (segment (start 210.5 82.5) (end 198 95) (width 1) (layer "B.Cu") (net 3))
 (segment (start 172.5 62) (end 182.5 62) (width 1) (layer "B.Cu") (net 3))
 (segment (start 182.5 62) (end 185.5 65) (width 1) (layer "B.Cu") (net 3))
 (segment (start 185.55 64.95) (end 195.95 64.95) (width 1) (layer "B.Cu") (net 3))
 (segment (start 195.95 64.95) (end 198 67) (width 1) (layer "B.Cu") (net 3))
 (segment (start 169.5 59) (end 172.5 62) (width 1) (layer "B.Cu") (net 3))
 (segment (start 198 111) (end 198 114) (width 1) (layer "B.Cu") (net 3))
 (segment (start 187.262742 42.5) (end 169.5 42.5) (width 1) (layer "B.Cu") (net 3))
 (segment (start 169.5 42.5) (end 169.5 59) (width 1) (layer "B.Cu") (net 3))
 (segment (start 198 79.5) (end 198 82.5) (width 1) (layer "B.Cu") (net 3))
 (segment (start 187.762742 42) (end 187.262742 42.5) (width 1) (layer "B.Cu") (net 3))
 (segment (start 210.5 98.5) (end 198 111) (width 1) (layer "B.Cu") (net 3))
 (segment (start 192.86 37.14) (end 188 42) (width 1) (layer "B.Cu") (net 3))
 (segment (start 192.86 35) (end 192.86 37.14) (width 1) (layer "B.Cu") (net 3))
 (segment (start 190.32 35) (end 190.32 37.18) (width 1) (layer "B.Cu") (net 5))
 (segment (start 181.25 95) (end 181.25 98.5) (width 1) (layer "B.Cu") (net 5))
 (segment (start 166.5 41.5) (end 166.5 59) (width 1) (layer "B.Cu") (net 5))
 (segment (start 171.5 64) (end 178.25 64) (width 1) (layer "B.Cu") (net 5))
 (segment (start 181.25 79.5) (end 181.25 82.5) (width 1) (layer "B.Cu") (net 5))
 (segment (start 167.5 40.5) (end 166.5 41.5) (width 1) (layer "B.Cu") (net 5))
 (segment (start 181.25 111) (end 181.25 114) (width 1) (layer "B.Cu") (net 5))
 (segment (start 190.32 37.18) (end 187 40.5) (width 1) (layer "B.Cu") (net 5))
 (segment (start 178.25 64) (end 181.25 67) (width 1) (layer "B.Cu") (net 5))
 (segment (start 193.75 67) (end 181.25 79.5) (width 1) (layer "B.Cu") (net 5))
 (segment (start 187 40.5) (end 167.5 40.5) (width 1) (layer "B.Cu") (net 5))
 (segment (start 166.5 59) (end 171.5 64) (width 1) (layer "B.Cu") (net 5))
 (segment (start 193.75 82.5) (end 181.25 95) (width 1) (layer "B.Cu") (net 5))
 (segment (start 193.75 98.5) (end 181.25 111) (width 1) (layer "B.Cu") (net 5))
 (segment (start 205 50) (end 202 47) (width 1) (layer "F.Cu") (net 6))
 (segment (start 207.5 77) (end 205 74.5) (width 1) (layer "F.Cu") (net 6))
 (segment (start 205 74.5) (end 205 59) (width 1) (layer "F.Cu") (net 6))
 (segment (start 205 59) (end 205 50) (width 1) (layer "F.Cu") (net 6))
 (via (at 202 47) (size 2.5) (drill 0.3) (layers "F.Cu" "B.Cu") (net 6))
 (via (at 207.5 77) (size 2.5) (drill 0.3) (layers "F.Cu" "B.Cu") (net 6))
 (segment (start 164.75 119) (end 178.2 105.55) (width 1) (layer "B.Cu") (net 6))
 (segment (start 182.95 105.55) (end 198.95 89.55) (width 1) (layer "B.Cu") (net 6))
 (segment (start 202 47) (end 203.02 45.98) (width 1) (layer "B.Cu") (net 6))
 (segment (start 193.75 119) (end 198 119) (width 1) (layer "B.Cu") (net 6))
 (segment (start 178.2 105.55) (end 182.95 105.55) (width 1) (layer "B.Cu") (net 6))
 (segment (start 207.5 81.549138) (end 207.5 77) (width 1) (layer "B.Cu") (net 6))
 (segment (start 199.499138 89.55) (end 207.5 81.549138) (width 1) (layer "B.Cu") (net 6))
 (segment (start 203.02 45.98) (end 203.02 35) (width 1) (layer "B.Cu") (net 6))
 (segment (start 198.95 89.55) (end 199.499138 89.55) (width 1) (layer "B.Cu") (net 6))
 (segment (start 177.25 119) (end 181.25 119) (width 1) (layer "B.Cu") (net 6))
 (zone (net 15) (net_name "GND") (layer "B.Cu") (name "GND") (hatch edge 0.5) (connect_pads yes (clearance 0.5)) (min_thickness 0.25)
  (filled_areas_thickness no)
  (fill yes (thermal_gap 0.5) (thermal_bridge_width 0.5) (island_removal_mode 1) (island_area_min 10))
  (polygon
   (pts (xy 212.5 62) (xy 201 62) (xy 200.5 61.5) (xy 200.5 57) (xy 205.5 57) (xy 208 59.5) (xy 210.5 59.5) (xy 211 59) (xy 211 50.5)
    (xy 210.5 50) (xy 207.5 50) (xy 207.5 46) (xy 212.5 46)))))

